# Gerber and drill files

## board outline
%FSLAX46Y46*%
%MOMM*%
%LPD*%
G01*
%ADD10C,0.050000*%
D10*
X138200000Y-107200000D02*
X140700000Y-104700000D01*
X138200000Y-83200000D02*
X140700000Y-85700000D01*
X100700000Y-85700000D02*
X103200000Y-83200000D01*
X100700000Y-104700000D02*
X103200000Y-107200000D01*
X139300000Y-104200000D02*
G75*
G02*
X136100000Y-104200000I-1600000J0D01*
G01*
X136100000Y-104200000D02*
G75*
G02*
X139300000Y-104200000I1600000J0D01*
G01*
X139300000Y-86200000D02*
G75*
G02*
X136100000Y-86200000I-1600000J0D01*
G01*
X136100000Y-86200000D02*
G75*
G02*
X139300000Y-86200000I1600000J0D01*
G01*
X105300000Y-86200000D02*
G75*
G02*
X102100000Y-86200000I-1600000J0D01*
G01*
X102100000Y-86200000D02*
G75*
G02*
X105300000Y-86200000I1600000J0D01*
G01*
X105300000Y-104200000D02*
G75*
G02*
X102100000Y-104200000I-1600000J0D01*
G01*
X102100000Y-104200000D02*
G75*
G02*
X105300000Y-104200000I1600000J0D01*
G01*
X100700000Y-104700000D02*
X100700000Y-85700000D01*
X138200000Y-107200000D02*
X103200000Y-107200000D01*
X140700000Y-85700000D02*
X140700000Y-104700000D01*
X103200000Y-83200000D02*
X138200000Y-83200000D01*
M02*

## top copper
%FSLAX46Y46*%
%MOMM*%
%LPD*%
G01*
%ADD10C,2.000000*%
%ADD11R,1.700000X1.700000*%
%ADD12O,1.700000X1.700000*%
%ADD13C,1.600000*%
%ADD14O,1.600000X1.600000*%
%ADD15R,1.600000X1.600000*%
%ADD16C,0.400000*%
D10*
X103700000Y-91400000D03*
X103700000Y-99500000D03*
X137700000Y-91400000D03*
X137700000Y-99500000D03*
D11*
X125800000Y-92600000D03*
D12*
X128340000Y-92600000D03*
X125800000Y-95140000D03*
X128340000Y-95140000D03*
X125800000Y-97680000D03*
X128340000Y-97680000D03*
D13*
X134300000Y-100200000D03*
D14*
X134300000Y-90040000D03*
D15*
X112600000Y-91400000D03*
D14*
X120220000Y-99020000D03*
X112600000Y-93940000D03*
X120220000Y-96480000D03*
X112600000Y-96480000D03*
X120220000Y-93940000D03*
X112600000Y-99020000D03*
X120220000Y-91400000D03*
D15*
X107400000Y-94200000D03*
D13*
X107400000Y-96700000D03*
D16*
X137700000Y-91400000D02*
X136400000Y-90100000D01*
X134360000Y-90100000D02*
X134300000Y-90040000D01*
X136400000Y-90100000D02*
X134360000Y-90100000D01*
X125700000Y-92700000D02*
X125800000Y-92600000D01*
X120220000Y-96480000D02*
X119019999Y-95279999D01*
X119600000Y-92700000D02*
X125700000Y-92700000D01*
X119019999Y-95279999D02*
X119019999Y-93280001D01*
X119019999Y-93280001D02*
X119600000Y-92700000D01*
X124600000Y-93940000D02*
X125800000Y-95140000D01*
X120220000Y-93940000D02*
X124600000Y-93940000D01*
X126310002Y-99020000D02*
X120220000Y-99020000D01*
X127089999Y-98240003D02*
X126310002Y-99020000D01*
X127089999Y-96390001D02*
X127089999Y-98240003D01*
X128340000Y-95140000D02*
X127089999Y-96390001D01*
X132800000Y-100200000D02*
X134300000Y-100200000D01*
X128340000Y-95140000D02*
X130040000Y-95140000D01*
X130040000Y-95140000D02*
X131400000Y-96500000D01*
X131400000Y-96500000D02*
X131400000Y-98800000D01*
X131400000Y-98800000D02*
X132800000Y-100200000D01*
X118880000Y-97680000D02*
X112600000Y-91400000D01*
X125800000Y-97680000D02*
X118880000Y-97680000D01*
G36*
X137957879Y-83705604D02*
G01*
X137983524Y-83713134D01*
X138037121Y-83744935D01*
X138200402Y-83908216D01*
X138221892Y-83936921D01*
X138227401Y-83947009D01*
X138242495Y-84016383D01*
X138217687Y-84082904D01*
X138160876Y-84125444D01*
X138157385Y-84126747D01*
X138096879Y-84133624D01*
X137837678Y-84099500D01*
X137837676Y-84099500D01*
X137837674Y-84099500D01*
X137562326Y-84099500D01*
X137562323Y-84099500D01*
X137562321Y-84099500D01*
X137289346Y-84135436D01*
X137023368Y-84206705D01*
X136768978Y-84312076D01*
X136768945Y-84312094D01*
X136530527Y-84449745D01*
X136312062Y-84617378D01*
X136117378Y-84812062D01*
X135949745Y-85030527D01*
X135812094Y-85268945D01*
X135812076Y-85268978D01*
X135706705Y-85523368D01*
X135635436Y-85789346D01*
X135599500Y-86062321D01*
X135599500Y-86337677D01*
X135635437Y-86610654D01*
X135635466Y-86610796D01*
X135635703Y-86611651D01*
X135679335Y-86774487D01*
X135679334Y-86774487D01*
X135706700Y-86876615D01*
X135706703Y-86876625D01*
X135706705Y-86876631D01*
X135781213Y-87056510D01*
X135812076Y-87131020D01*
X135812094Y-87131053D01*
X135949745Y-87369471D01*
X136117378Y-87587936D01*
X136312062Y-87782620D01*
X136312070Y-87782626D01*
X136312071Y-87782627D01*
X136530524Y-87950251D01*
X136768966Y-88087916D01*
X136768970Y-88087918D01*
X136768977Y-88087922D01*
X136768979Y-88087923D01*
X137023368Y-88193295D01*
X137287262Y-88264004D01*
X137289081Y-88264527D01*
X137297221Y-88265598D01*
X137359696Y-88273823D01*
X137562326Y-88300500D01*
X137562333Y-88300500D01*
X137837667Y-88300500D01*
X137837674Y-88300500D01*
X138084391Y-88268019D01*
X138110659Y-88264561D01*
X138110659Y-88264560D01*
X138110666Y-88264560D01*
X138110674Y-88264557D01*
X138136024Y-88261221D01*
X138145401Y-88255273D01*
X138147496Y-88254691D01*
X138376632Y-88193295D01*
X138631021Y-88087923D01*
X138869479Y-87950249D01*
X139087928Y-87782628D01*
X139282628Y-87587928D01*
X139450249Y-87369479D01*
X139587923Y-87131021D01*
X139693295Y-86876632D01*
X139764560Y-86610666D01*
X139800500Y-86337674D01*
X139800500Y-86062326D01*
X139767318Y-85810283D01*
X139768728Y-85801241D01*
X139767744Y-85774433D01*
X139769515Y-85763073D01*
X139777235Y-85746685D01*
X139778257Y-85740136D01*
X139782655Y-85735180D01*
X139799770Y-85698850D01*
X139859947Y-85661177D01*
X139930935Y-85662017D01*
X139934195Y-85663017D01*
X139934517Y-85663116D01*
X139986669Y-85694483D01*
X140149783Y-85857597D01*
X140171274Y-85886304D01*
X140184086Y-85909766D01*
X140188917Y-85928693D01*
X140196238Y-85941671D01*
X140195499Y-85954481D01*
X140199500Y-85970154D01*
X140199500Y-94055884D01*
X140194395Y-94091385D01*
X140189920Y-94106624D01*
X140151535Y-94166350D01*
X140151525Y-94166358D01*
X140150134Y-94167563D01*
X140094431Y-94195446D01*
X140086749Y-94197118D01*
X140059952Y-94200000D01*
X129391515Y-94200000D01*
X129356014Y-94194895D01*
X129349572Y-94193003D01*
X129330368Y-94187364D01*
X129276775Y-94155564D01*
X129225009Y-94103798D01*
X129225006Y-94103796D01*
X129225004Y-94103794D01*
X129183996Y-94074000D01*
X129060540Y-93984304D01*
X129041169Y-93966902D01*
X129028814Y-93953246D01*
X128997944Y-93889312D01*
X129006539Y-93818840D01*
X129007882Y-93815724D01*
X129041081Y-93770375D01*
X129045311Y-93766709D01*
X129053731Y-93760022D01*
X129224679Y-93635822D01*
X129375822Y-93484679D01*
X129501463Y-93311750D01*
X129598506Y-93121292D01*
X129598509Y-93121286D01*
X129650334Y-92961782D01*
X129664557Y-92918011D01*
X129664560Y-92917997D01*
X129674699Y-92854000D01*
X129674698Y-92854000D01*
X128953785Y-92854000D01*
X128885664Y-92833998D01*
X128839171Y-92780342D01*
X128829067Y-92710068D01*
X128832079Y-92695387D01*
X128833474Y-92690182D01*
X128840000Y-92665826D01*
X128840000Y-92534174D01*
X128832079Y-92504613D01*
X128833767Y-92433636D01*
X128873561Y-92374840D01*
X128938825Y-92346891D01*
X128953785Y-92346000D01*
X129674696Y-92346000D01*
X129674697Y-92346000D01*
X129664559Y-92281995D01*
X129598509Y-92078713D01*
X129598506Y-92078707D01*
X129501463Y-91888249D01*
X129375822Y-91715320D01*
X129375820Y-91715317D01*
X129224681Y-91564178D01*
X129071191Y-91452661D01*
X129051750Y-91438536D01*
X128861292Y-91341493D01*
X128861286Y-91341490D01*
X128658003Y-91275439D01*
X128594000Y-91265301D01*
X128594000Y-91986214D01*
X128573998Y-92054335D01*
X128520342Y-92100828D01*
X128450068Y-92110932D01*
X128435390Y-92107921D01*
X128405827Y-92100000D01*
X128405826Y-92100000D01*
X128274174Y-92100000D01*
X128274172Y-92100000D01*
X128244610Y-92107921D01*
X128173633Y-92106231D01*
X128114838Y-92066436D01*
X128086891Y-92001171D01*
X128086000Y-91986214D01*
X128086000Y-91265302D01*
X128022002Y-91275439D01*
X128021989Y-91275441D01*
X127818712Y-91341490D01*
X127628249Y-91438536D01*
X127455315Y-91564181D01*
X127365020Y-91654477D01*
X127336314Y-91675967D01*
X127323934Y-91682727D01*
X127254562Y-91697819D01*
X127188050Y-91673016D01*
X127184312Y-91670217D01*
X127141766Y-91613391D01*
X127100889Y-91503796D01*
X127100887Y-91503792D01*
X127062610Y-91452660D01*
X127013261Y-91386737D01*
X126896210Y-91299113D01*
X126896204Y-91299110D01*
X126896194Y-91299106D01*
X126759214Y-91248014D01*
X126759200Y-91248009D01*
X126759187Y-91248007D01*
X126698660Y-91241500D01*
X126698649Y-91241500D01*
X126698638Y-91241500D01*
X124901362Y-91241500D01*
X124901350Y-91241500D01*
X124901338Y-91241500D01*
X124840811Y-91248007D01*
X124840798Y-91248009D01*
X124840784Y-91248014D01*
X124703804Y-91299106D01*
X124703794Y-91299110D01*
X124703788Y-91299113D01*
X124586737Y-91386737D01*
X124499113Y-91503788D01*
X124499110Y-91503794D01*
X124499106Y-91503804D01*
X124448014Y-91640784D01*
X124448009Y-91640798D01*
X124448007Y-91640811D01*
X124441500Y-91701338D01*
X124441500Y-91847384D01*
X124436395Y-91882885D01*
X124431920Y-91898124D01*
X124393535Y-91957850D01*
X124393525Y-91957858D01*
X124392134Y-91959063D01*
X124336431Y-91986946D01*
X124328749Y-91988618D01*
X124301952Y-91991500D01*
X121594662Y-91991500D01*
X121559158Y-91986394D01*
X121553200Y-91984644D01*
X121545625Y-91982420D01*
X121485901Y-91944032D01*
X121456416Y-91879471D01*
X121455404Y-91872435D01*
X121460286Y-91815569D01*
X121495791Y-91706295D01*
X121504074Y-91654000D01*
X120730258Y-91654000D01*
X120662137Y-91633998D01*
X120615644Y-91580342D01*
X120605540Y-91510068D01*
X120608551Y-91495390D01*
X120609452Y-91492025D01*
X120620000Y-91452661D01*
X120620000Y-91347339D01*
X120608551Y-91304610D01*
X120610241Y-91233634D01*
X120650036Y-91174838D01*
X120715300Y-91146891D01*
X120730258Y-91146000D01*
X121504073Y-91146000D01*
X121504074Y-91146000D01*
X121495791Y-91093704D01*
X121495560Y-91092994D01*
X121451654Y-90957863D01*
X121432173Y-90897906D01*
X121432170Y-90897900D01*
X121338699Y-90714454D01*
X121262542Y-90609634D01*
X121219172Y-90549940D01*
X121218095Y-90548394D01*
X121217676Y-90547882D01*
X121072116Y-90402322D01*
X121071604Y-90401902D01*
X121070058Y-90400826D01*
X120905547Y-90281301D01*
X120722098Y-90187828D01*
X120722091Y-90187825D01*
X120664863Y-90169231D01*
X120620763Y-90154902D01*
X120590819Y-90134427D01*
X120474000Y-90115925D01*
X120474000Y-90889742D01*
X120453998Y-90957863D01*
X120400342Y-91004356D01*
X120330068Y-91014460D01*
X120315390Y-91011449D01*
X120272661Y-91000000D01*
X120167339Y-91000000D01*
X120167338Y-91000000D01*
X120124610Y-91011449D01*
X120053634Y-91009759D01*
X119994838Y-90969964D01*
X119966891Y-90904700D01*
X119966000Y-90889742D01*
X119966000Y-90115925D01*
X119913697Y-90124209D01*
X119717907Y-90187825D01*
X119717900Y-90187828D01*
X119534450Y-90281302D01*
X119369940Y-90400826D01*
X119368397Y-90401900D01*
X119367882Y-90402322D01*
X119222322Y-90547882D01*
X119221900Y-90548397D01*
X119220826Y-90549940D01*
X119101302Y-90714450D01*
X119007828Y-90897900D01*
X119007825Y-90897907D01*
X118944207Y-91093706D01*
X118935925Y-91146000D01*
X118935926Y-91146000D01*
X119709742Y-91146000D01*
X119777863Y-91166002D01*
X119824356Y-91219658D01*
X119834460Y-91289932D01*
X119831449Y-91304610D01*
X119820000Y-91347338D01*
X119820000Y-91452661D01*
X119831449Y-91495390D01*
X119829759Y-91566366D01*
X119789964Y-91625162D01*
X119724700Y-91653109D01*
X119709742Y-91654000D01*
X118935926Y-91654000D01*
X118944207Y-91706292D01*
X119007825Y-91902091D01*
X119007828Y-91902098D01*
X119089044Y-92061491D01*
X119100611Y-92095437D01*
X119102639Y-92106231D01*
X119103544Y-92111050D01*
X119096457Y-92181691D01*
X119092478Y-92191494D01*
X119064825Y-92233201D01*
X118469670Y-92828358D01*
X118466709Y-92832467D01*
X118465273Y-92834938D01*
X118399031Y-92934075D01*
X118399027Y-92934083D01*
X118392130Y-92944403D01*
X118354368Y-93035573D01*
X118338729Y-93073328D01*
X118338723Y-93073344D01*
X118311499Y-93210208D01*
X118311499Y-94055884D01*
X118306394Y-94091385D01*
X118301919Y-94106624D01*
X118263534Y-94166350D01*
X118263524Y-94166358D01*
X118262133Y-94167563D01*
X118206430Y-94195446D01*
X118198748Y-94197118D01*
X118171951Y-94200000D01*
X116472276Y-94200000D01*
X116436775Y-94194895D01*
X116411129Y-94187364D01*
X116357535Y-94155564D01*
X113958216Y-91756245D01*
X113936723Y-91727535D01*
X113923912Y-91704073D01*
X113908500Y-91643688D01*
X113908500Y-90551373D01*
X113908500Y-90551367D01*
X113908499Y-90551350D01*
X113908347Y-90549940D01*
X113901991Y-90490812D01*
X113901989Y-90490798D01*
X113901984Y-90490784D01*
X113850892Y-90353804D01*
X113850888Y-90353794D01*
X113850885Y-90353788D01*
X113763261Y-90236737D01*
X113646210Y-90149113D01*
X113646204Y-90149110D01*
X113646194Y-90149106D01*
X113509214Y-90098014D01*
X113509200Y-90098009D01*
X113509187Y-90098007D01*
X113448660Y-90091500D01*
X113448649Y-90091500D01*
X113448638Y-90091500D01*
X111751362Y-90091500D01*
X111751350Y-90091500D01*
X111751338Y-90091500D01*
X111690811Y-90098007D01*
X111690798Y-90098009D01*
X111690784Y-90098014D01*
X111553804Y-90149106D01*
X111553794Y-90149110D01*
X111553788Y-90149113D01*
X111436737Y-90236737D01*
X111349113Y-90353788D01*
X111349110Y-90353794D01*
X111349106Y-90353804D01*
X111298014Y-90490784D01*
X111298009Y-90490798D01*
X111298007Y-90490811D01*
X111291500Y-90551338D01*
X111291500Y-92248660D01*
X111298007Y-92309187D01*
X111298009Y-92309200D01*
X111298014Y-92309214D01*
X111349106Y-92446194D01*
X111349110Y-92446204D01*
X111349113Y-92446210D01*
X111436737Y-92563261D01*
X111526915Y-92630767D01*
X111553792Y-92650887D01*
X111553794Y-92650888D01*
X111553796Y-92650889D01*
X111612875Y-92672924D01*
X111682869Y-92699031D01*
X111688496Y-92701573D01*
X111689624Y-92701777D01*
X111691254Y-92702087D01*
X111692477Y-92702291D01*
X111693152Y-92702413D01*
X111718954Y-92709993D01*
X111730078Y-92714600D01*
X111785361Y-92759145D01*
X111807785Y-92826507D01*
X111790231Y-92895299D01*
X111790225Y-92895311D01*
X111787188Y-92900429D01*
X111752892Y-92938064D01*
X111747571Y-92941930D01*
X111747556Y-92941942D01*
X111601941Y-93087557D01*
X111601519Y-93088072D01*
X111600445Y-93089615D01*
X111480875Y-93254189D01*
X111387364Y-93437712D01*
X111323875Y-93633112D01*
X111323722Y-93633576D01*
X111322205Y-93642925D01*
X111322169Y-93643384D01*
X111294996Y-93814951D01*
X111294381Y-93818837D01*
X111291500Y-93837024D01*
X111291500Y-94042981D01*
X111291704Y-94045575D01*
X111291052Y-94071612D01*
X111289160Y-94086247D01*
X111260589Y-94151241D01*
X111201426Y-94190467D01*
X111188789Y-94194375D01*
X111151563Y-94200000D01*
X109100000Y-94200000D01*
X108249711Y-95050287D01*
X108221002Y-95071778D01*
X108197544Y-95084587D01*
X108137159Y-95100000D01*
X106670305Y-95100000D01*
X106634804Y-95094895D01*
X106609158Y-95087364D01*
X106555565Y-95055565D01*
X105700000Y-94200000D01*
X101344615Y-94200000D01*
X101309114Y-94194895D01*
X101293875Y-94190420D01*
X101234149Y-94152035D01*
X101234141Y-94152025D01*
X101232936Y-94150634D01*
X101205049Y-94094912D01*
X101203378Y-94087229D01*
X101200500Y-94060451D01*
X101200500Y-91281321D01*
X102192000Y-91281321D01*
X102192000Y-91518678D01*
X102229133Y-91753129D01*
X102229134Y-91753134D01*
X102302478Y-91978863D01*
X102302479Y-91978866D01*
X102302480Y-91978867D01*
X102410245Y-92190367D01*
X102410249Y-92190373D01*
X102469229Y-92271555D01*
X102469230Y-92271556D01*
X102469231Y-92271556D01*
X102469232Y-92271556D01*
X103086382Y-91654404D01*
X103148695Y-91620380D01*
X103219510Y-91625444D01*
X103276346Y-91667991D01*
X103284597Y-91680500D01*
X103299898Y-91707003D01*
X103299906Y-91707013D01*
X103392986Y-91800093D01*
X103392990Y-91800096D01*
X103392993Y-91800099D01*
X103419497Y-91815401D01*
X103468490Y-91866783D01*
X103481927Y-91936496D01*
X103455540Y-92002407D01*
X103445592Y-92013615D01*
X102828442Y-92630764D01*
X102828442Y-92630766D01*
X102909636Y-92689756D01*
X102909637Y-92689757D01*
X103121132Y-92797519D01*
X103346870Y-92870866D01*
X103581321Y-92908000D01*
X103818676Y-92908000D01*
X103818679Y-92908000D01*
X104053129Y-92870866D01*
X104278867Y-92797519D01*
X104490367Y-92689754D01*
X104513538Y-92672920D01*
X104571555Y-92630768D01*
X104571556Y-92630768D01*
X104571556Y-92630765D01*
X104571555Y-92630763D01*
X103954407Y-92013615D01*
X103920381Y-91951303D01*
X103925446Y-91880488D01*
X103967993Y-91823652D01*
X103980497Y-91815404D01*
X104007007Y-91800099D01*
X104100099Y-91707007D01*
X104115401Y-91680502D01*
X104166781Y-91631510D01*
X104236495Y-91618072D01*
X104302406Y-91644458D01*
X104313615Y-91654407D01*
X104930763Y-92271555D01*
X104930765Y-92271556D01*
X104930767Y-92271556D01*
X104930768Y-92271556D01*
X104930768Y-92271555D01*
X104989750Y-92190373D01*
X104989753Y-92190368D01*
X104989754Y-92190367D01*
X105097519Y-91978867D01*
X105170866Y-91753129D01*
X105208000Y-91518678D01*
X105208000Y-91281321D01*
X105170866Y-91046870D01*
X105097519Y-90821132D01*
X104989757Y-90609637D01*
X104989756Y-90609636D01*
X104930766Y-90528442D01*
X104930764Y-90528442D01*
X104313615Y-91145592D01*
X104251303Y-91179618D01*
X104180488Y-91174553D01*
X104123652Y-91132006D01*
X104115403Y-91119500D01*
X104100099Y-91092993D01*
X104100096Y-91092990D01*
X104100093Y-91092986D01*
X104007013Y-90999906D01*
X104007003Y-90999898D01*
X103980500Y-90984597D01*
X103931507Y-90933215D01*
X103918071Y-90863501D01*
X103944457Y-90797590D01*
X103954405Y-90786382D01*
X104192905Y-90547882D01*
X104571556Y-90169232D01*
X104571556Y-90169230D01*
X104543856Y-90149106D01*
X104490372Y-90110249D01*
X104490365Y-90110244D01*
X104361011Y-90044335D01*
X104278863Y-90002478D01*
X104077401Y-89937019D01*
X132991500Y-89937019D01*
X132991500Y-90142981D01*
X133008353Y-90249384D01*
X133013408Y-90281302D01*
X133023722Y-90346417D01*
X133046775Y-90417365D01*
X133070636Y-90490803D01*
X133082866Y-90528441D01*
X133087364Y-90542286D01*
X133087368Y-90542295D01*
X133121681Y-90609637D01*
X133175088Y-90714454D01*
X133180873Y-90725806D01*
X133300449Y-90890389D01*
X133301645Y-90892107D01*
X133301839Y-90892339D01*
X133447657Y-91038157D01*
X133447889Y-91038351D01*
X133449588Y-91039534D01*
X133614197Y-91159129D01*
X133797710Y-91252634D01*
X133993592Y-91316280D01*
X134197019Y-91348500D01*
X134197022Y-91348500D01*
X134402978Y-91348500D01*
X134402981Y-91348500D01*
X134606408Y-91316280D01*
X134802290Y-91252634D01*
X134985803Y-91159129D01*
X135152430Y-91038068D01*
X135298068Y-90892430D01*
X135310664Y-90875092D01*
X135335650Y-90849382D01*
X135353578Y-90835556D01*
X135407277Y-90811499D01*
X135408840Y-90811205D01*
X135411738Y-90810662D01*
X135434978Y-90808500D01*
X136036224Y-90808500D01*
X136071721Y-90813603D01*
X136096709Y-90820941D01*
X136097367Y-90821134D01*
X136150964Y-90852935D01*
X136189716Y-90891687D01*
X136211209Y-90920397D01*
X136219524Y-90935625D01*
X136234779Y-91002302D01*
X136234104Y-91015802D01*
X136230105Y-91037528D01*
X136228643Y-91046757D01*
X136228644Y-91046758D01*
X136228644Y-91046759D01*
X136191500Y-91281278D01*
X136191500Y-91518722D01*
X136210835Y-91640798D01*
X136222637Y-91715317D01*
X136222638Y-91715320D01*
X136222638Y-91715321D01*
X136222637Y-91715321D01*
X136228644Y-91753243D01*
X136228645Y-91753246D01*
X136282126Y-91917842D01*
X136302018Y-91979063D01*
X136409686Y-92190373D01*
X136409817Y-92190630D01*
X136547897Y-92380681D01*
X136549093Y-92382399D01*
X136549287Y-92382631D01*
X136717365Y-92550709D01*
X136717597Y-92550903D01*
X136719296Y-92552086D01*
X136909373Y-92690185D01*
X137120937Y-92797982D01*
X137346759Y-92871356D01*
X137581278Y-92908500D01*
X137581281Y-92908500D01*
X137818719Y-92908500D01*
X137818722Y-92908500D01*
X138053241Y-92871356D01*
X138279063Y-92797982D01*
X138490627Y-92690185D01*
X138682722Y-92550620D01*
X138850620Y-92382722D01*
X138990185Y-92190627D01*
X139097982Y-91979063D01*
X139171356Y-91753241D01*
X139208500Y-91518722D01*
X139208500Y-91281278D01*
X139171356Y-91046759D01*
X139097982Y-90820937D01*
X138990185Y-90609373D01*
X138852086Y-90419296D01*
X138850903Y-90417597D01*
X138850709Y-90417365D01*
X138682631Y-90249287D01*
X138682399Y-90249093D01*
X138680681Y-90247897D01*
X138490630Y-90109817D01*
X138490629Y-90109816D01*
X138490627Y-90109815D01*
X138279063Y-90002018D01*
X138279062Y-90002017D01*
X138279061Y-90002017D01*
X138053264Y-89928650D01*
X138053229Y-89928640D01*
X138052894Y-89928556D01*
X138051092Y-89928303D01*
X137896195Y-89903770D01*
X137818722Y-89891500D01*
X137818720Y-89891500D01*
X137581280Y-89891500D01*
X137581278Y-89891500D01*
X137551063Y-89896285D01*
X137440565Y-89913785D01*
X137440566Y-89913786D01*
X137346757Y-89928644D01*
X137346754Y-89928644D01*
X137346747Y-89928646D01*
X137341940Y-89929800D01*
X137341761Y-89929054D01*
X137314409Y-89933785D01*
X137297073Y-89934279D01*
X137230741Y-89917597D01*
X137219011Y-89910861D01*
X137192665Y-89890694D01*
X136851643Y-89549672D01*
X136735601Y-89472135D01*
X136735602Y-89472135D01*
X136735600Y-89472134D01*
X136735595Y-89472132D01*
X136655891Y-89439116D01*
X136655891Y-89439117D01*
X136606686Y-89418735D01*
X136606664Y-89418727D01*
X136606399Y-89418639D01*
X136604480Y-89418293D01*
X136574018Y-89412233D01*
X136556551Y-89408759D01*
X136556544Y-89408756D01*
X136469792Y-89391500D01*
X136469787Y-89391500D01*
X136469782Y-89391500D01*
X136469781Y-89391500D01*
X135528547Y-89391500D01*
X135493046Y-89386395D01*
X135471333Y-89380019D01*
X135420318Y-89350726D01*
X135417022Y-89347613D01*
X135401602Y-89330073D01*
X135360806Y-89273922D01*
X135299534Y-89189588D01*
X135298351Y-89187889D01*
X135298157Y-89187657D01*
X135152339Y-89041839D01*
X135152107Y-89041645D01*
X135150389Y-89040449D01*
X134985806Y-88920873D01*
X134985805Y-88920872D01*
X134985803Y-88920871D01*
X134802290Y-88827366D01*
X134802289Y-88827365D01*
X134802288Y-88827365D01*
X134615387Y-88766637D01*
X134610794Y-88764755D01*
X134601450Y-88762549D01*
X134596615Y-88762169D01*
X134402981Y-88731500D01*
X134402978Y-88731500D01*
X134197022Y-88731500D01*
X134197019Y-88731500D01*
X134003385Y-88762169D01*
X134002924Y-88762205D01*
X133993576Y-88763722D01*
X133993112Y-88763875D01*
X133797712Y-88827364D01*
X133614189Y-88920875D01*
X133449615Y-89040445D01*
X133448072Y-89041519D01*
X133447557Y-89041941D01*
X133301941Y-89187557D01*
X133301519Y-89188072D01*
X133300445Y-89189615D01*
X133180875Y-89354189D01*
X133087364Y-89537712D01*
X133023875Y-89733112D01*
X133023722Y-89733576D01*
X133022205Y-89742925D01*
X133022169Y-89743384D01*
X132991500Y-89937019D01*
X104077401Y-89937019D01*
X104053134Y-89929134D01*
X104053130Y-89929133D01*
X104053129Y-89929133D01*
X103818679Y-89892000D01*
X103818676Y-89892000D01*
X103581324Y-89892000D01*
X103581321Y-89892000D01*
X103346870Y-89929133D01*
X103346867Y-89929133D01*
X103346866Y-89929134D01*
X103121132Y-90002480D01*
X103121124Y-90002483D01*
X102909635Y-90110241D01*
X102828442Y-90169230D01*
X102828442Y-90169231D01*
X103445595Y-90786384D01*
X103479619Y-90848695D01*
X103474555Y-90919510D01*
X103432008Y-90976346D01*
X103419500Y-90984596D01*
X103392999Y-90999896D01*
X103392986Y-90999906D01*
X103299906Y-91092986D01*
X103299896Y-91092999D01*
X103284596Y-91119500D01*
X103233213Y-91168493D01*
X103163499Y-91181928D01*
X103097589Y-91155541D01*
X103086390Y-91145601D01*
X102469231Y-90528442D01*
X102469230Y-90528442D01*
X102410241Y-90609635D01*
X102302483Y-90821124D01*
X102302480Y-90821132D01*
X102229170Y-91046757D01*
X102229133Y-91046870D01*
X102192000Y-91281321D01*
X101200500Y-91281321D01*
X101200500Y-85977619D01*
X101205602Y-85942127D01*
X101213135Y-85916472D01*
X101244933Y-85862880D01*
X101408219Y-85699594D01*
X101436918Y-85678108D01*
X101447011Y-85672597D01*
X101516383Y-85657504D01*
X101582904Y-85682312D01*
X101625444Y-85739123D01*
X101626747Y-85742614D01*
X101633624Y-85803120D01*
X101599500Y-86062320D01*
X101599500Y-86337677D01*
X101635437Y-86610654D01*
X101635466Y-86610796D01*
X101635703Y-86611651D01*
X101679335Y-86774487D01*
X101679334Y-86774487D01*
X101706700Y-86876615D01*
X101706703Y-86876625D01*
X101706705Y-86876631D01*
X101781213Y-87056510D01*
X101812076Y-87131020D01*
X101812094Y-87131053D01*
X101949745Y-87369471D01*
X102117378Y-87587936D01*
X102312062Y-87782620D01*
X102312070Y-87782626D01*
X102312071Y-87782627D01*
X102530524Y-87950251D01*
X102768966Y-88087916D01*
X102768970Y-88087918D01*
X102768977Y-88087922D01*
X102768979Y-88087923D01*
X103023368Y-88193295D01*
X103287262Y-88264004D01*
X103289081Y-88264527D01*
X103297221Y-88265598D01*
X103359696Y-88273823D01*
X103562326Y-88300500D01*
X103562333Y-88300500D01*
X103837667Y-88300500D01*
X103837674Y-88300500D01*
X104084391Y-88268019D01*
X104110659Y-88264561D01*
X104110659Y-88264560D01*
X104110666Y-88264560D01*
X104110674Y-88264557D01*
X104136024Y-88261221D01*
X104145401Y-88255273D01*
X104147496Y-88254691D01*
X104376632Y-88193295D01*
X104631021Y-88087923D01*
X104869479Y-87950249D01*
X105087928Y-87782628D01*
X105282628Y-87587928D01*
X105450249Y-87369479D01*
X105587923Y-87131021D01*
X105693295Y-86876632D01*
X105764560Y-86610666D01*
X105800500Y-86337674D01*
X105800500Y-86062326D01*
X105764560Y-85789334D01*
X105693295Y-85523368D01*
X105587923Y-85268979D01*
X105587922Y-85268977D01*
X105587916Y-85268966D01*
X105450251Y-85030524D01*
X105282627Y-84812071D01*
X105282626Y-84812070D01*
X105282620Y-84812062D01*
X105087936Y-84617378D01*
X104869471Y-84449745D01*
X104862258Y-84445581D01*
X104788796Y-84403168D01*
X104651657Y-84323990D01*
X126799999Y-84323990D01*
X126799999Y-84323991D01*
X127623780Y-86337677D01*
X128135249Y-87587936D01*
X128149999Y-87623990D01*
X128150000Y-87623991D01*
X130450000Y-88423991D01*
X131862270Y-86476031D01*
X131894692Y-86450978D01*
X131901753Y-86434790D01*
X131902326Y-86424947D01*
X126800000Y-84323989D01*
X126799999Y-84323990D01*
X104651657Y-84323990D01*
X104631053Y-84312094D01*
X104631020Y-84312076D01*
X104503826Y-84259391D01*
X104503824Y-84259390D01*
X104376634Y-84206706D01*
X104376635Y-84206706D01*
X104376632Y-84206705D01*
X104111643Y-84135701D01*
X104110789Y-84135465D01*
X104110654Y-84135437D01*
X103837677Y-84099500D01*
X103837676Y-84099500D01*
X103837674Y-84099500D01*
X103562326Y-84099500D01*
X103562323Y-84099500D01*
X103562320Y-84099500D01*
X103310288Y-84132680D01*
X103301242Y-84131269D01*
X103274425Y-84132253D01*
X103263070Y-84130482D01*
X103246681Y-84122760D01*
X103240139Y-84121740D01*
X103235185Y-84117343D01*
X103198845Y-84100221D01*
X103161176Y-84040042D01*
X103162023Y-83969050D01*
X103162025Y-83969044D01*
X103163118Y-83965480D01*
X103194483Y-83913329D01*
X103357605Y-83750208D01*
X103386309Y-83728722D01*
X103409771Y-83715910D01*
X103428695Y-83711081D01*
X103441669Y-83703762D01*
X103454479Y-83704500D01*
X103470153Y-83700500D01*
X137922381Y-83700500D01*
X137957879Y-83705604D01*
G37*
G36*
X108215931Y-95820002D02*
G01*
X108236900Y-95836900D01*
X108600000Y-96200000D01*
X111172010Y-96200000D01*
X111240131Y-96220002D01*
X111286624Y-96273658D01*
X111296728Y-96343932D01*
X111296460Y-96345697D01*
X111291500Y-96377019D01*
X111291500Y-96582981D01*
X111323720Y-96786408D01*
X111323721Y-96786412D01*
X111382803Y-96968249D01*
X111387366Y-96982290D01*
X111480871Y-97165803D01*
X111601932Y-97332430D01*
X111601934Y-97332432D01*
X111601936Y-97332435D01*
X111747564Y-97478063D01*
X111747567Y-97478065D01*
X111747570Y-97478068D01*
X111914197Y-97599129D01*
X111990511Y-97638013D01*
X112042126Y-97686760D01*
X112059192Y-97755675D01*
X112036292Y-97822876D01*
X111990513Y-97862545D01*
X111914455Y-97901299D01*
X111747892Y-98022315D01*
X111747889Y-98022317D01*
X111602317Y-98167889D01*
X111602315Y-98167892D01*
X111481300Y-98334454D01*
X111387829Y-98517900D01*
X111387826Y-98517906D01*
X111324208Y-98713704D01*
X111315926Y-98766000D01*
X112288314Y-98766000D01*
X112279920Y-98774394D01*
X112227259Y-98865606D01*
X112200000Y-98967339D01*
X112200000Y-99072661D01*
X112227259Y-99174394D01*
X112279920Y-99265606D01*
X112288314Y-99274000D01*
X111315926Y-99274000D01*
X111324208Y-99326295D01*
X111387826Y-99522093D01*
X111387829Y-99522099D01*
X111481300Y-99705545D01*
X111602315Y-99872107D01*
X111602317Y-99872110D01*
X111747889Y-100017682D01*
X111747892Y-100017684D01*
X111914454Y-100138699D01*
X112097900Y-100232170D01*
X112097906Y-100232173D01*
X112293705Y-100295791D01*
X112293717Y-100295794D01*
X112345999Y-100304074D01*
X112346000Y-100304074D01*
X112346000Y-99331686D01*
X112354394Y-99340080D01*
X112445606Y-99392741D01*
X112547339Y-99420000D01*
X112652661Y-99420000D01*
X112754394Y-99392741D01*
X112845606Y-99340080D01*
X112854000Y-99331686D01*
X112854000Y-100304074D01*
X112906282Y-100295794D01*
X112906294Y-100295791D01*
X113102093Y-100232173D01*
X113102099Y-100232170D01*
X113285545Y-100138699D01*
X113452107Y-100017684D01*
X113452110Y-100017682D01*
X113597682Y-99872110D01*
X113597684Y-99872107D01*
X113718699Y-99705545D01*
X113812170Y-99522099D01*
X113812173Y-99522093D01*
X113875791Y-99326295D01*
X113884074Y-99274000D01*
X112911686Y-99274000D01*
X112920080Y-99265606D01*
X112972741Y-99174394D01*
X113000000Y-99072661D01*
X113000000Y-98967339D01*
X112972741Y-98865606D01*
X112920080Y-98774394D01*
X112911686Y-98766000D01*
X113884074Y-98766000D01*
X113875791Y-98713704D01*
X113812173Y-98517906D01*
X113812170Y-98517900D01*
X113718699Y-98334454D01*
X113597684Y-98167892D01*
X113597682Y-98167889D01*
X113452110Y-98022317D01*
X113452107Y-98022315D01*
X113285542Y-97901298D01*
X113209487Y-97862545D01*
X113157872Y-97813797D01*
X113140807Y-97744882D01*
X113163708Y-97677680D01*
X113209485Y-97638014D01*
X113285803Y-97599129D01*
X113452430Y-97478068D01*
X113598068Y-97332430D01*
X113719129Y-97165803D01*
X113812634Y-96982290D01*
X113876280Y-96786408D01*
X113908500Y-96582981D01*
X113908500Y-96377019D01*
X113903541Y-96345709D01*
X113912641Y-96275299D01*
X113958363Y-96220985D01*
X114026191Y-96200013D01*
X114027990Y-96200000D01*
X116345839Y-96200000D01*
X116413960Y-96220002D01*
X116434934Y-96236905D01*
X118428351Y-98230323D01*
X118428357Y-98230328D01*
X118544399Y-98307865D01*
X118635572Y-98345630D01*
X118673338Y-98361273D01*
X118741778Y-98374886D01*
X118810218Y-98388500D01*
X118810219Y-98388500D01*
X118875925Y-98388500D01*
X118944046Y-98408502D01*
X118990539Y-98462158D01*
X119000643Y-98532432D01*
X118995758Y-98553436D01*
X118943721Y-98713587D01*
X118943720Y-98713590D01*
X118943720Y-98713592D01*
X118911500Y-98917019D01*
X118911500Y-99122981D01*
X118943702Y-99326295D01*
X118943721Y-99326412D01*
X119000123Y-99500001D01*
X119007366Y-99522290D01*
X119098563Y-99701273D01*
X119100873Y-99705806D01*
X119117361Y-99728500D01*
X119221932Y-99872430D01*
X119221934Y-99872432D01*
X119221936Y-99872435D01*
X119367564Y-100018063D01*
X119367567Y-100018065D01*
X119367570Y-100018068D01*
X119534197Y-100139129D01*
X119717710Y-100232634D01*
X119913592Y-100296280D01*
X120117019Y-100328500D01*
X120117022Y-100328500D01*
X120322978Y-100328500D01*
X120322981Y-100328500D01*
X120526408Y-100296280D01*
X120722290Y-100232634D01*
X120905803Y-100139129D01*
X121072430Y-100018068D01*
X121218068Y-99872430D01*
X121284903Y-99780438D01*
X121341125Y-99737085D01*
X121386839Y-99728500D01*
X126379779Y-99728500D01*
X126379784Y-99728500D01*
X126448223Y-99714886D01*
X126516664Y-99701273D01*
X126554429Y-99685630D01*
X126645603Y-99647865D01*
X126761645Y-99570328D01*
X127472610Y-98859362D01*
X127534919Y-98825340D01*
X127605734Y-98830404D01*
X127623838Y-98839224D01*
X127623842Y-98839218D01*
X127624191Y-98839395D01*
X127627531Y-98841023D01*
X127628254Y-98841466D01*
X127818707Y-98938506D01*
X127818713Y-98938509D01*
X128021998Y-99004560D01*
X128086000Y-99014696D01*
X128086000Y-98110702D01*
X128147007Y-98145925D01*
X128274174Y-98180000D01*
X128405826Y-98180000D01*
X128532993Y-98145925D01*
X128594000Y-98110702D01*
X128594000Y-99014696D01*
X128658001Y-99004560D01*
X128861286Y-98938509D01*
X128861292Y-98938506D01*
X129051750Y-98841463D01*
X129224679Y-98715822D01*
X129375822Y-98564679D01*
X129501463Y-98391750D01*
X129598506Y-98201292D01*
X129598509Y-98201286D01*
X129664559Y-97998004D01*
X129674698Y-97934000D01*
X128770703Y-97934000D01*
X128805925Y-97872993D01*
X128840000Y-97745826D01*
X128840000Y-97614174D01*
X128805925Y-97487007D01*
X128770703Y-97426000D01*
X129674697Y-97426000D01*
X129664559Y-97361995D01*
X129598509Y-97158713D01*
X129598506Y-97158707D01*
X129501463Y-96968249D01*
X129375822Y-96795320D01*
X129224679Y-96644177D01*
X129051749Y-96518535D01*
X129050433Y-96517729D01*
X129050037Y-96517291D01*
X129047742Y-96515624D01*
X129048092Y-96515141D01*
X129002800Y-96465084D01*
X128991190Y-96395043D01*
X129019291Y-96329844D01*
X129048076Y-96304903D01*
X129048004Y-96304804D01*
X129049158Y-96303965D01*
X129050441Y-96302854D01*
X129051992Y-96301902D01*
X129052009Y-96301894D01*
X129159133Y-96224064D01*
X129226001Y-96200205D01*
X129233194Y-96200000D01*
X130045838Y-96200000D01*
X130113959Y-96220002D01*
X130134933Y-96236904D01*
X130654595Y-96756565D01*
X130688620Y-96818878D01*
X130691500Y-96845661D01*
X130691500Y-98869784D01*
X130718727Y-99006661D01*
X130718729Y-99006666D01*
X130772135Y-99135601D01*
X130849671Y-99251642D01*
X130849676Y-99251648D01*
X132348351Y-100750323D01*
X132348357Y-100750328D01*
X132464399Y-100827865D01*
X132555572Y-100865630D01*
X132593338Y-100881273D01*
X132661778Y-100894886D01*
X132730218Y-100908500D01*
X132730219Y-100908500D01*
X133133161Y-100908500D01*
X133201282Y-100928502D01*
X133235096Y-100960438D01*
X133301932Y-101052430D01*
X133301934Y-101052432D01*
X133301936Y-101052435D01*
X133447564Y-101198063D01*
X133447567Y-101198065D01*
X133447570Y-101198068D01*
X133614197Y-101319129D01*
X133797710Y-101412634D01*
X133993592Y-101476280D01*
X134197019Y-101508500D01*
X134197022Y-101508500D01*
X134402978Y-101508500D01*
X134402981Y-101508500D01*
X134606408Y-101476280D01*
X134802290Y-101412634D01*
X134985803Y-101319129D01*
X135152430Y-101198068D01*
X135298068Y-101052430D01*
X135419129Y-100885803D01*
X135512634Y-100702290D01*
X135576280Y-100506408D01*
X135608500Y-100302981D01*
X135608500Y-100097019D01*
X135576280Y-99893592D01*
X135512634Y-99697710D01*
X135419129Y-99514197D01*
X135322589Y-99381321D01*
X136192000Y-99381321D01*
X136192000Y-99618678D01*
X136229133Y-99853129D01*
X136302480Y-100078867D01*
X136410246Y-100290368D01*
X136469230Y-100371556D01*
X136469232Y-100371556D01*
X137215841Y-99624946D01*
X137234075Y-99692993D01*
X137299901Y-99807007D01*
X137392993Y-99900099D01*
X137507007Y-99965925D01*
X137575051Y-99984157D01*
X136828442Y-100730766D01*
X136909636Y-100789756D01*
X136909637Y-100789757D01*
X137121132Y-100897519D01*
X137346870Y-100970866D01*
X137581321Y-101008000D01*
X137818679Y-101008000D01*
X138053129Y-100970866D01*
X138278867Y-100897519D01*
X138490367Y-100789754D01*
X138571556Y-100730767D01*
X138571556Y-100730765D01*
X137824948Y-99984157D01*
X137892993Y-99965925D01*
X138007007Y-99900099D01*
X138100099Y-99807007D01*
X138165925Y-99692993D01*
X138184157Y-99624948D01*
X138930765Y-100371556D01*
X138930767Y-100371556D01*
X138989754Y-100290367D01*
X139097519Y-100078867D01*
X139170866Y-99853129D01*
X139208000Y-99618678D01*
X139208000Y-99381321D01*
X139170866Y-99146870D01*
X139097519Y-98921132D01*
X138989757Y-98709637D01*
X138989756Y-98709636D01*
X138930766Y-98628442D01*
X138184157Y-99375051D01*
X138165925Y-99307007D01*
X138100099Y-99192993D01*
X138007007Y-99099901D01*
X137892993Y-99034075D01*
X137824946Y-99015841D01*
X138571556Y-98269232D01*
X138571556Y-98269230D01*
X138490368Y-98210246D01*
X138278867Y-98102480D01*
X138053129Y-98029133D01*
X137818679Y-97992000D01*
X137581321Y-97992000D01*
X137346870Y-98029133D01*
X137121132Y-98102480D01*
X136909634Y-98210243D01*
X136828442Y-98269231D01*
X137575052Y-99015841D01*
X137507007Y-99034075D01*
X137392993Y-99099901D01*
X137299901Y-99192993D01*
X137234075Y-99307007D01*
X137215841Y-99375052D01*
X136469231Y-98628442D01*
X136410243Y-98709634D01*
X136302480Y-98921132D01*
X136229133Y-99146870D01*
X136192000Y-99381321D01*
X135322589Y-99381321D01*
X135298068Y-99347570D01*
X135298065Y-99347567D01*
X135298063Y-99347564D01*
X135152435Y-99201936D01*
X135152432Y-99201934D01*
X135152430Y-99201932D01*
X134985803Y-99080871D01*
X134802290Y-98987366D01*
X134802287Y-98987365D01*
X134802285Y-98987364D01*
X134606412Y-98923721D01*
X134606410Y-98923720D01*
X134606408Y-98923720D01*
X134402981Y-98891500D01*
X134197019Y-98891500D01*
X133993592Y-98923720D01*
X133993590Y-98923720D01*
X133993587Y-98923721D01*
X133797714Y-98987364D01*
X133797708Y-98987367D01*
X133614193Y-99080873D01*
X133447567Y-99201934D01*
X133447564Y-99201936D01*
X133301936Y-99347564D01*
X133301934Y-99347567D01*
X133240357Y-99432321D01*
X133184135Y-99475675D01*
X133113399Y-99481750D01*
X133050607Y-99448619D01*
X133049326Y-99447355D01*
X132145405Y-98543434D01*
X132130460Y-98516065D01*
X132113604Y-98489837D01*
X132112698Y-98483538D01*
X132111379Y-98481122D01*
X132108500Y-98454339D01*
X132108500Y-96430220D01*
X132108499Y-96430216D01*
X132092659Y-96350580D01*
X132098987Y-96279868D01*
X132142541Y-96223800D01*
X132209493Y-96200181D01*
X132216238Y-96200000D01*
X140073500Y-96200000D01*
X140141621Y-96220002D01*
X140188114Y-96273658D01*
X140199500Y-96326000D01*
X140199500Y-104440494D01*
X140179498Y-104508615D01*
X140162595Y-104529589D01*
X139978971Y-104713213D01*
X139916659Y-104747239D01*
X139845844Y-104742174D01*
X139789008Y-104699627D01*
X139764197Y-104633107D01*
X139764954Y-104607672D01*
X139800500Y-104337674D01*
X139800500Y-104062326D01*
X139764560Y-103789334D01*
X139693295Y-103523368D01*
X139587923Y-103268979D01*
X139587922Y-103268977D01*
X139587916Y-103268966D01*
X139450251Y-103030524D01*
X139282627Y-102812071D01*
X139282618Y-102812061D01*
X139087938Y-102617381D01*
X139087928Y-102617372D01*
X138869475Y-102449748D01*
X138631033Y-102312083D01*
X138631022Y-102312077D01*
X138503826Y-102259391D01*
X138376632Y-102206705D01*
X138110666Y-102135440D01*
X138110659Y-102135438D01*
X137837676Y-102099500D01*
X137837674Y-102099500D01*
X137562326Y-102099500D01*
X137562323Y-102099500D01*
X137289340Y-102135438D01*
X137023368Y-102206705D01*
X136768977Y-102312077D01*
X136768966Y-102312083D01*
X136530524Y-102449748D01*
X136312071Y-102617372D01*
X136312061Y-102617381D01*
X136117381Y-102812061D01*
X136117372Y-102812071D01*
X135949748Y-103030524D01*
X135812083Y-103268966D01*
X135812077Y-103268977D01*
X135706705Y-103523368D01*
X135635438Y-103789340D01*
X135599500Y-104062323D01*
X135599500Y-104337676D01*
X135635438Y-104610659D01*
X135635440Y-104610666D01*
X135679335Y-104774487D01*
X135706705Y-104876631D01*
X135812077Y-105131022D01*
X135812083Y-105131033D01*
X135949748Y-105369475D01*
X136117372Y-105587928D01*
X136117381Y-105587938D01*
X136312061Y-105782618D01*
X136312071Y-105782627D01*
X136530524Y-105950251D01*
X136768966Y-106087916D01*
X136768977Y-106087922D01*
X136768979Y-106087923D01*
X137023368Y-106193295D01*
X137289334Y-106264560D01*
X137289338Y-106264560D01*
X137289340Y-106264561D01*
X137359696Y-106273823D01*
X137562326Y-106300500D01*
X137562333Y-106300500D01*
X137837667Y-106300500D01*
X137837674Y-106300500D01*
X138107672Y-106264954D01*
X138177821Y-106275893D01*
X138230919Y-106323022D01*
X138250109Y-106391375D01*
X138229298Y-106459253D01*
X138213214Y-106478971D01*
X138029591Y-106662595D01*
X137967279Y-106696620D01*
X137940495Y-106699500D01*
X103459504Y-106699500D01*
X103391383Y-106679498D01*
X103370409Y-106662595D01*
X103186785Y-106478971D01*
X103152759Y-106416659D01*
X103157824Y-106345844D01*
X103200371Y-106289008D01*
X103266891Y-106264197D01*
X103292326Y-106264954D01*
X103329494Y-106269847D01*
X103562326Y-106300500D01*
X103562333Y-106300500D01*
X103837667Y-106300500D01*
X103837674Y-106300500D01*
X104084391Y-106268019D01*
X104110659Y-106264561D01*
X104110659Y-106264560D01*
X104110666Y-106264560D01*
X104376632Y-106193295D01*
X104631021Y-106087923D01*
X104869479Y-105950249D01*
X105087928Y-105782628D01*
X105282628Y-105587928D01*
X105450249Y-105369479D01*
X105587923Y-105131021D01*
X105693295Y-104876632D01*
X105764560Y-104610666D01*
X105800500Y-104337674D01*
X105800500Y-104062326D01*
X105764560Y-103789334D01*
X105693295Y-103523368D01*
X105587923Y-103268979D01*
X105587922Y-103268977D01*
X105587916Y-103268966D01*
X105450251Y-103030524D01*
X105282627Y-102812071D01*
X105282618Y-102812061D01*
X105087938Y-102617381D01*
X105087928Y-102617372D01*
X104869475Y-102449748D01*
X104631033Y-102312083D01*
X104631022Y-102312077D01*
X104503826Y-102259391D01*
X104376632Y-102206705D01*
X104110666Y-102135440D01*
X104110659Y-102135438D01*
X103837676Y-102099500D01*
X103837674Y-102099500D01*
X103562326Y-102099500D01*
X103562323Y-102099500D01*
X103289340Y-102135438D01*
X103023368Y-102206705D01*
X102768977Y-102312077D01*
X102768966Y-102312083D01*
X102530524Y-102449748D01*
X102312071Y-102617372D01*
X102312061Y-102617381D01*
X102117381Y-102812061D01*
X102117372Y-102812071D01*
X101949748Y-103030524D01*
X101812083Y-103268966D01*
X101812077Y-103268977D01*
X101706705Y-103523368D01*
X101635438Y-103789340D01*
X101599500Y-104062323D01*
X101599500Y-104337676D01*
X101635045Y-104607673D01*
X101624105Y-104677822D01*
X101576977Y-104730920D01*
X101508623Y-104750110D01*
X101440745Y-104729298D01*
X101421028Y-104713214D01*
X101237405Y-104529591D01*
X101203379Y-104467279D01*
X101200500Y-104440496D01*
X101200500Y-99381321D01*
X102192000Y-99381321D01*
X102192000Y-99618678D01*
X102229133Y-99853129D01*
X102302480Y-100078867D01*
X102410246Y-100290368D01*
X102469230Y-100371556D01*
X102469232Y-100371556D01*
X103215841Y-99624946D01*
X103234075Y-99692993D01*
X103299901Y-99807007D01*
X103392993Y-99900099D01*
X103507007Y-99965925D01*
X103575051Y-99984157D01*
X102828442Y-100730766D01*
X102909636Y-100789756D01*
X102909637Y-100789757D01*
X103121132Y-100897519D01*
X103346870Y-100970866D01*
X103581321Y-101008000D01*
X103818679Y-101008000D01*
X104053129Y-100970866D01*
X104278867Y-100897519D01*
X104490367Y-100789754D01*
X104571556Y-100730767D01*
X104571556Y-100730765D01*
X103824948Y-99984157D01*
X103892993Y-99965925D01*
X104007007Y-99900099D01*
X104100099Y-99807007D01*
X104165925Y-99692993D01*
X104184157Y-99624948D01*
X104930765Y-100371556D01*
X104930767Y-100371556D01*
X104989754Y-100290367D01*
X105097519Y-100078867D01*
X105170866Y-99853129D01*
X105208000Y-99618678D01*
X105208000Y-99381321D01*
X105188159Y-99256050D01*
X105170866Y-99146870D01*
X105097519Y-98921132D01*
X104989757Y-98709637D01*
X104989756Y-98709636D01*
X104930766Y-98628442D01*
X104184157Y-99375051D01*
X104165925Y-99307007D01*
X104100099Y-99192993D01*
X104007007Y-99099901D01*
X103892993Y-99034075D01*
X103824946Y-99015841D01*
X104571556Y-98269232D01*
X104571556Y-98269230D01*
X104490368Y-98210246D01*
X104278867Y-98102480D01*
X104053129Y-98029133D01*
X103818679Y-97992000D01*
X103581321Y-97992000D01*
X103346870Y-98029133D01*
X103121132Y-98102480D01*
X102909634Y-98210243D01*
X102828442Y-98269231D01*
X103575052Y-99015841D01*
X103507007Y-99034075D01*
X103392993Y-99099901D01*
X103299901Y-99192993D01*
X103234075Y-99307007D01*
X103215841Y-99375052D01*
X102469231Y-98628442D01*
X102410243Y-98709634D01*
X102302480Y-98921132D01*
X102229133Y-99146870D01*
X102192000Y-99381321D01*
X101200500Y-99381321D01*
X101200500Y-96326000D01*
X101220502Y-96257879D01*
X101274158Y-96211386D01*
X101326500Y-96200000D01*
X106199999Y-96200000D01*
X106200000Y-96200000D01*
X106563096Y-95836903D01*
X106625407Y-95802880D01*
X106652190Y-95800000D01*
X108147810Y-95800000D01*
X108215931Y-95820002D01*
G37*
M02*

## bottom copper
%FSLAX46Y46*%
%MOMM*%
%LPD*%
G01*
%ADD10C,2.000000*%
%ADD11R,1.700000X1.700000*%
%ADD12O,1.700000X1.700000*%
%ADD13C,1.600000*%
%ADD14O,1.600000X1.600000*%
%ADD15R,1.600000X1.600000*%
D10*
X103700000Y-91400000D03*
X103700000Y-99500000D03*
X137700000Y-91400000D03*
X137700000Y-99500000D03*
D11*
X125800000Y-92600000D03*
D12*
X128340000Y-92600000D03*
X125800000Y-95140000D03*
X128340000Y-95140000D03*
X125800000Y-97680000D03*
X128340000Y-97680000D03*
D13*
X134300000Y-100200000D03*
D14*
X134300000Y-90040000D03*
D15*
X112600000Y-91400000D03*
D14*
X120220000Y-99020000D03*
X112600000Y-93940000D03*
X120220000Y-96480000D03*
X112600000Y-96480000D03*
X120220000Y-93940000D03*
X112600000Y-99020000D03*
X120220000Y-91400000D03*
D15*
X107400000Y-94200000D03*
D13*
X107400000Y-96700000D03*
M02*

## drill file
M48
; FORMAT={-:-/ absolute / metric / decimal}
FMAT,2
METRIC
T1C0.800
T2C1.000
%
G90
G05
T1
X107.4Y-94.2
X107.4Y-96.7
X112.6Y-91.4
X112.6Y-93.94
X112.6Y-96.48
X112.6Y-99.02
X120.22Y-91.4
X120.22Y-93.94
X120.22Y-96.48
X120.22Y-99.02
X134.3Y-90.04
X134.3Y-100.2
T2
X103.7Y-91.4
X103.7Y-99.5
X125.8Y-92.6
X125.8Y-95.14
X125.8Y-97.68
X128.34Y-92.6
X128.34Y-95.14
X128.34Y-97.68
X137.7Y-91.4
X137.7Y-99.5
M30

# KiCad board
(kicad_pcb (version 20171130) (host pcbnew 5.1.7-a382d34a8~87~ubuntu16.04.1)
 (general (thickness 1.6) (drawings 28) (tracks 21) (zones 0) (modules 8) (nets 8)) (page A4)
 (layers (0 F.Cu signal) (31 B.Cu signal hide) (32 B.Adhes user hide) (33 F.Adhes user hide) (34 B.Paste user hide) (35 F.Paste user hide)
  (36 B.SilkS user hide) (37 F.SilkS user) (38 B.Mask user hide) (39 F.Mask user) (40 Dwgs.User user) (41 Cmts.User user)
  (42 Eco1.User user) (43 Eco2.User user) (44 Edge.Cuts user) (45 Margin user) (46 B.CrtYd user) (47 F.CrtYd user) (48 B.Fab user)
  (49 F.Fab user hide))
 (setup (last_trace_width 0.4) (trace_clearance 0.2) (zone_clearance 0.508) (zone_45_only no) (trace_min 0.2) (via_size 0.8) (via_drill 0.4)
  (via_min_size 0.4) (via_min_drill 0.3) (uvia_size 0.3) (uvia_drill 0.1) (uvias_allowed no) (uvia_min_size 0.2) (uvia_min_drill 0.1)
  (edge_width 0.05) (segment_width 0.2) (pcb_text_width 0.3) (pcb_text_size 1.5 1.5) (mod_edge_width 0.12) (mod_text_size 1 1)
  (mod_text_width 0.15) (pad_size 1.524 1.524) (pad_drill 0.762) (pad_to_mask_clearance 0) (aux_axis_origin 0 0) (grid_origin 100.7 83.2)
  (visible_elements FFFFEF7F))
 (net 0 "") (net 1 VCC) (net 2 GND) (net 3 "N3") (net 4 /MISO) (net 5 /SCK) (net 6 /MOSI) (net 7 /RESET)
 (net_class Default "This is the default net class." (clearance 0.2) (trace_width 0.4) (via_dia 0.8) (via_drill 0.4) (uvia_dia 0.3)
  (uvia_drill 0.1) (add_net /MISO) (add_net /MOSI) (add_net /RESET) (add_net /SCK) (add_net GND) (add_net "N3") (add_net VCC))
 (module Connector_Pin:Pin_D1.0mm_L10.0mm (layer F.Cu) (at 103.7 91.4)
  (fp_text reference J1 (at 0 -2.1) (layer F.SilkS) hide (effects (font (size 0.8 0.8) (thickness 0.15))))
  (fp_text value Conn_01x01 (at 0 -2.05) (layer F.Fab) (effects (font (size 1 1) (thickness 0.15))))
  (pad 1 thru_hole circle (at 0 0) (size 2 2) (drill 1) (layers *.Cu *.Mask) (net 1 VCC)))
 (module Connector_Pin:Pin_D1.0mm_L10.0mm (layer F.Cu) (at 103.7 99.5)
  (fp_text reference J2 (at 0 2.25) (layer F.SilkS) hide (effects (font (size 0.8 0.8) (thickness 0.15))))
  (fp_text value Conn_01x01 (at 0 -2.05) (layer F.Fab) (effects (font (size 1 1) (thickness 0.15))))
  (pad 1 thru_hole circle (at 0 0) (size 2 2) (drill 1) (layers *.Cu *.Mask) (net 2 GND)))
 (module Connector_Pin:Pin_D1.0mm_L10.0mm (layer F.Cu) (at 137.7 91.4)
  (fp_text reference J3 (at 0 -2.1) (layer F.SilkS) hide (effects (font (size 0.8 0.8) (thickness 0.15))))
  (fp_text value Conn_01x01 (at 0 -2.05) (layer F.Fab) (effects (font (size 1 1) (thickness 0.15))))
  (pad 1 thru_hole circle (at 0 0) (size 2 2) (drill 1) (layers *.Cu *.Mask) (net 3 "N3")))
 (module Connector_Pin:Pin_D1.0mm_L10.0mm (layer F.Cu) (at 137.7 99.5)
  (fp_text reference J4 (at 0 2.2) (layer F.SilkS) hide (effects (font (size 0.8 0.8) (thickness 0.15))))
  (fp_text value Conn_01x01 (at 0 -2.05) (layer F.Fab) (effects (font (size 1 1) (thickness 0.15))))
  (pad 1 thru_hole circle (at 0 0) (size 2 2) (drill 1) (layers *.Cu *.Mask) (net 2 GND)))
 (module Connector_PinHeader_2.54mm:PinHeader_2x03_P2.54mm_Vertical (layer F.Cu) (at 125.8 92.6)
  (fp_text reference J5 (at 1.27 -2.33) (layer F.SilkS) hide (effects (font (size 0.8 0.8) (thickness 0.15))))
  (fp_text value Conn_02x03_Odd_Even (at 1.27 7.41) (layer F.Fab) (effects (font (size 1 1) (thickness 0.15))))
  (pad 1 thru_hole rect (at 0 0) (size 1.7 1.7) (drill 1) (layers *.Cu *.Mask) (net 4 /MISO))
  (pad 2 thru_hole oval (at 2.54 0) (size 1.7 1.7) (drill 1) (layers *.Cu *.Mask) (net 1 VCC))
  (pad 3 thru_hole oval (at 0 2.54) (size 1.7 1.7) (drill 1) (layers *.Cu *.Mask) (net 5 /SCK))
  (pad 4 thru_hole oval (at 2.54 2.54) (size 1.7 1.7) (drill 1) (layers *.Cu *.Mask) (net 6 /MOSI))
  (pad 5 thru_hole oval (at 0 5.08) (size 1.7 1.7) (drill 1) (layers *.Cu *.Mask) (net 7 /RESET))
  (pad 6 thru_hole oval (at 2.54 5.08) (size 1.7 1.7) (drill 1) (layers *.Cu *.Mask) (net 2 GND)))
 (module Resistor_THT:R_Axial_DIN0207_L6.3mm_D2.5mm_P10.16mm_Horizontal (layer F.Cu) (at 134.3 100.2 90)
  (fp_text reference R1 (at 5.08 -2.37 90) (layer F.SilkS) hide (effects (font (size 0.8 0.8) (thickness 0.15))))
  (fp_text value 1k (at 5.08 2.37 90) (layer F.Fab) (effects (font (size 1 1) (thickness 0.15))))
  (pad 1 thru_hole circle (at 0 0 90) (size 1.6 1.6) (drill 0.8) (layers *.Cu *.Mask) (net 6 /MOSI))
  (pad 2 thru_hole oval (at 10.16 0 90) (size 1.6 1.6) (drill 0.8) (layers *.Cu *.Mask) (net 3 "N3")))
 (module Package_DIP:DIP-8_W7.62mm (layer F.Cu) (at 112.6 91.4)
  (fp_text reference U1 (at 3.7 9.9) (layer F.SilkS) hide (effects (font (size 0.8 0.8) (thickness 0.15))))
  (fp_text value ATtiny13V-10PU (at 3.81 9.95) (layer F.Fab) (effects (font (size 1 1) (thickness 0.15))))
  (pad 1 thru_hole rect (at 0 0) (size 1.6 1.6) (drill 0.8) (layers *.Cu *.Mask) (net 7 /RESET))
  (pad 5 thru_hole oval (at 7.62 7.62) (size 1.6 1.6) (drill 0.8) (layers *.Cu *.Mask) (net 6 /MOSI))
  (pad 2 thru_hole oval (at 0 2.54) (size 1.6 1.6) (drill 0.8) (layers *.Cu *.Mask))
  (pad 6 thru_hole oval (at 7.62 5.08) (size 1.6 1.6) (drill 0.8) (layers *.Cu *.Mask) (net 4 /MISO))
  (pad 3 thru_hole oval (at 0 5.08) (size 1.6 1.6) (drill 0.8) (layers *.Cu *.Mask))
  (pad 7 thru_hole oval (at 7.62 2.54) (size 1.6 1.6) (drill 0.8) (layers *.Cu *.Mask) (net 5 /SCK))
  (pad 4 thru_hole oval (at 0 7.62) (size 1.6 1.6) (drill 0.8) (layers *.Cu *.Mask) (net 2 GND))
  (pad 8 thru_hole oval (at 7.62 0) (size 1.6 1.6) (drill 0.8) (layers *.Cu *.Mask) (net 1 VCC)))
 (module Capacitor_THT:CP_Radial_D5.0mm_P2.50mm (layer F.Cu) (at 107.4 94.2 270) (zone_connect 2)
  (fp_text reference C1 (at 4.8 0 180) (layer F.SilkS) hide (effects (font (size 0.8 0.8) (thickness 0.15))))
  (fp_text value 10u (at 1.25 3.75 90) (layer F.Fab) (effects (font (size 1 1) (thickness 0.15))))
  (pad 1 thru_hole rect (at 0 0 270) (size 1.6 1.6) (drill 0.8) (layers *.Cu *.Mask) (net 1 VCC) (zone_connect 2))
  (pad 2 thru_hole circle (at 2.5 0 270) (size 1.6 1.6) (drill 0.8) (layers *.Cu *.Mask) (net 2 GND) (zone_connect 2)))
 (gr_line (start 138.2 107.2) (end 140.7 104.7) (layer Edge.Cuts) (width 0.05))
 (gr_line (start 138.2 83.2) (end 140.7 85.7) (layer Edge.Cuts) (width 0.05))
 (gr_line (start 100.7 85.7) (end 103.2 83.2) (layer Edge.Cuts) (width 0.05))
 (gr_line (start 100.7 104.7) (end 103.2 107.2) (layer Edge.Cuts) (width 0.05))
 (gr_circle (center 137.7 104.2) (end 139.3 104.2) (layer Edge.Cuts) (width 0.05))
 (gr_circle (center 137.7 86.2) (end 139.3 86.2) (layer Edge.Cuts) (width 0.05))
 (gr_circle (center 103.7 86.2) (end 105.3 86.2) (layer Edge.Cuts) (width 0.05))
 (gr_circle (center 103.7 104.2) (end 105.3 104.2) (layer Edge.Cuts) (width 0.05))
 (gr_line (start 100.7 104.7) (end 100.7 85.7) (layer Edge.Cuts) (width 0.05))
 (gr_line (start 138.2 107.2) (end 103.2 107.2) (layer Edge.Cuts) (width 0.05))
 (gr_line (start 140.7 85.7) (end 140.7 104.7) (layer Edge.Cuts) (width 0.05))
 (gr_line (start 103.2 83.2) (end 138.2 83.2) (layer Edge.Cuts) (width 0.05))
 (segment (start 137.7 91.4) (end 136.4 90.1) (width 0.4) (layer F.Cu) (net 3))
 (segment (start 134.36 90.1) (end 134.3 90.04) (width 0.4) (layer F.Cu) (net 3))
 (segment (start 136.4 90.1) (end 134.36 90.1) (width 0.4) (layer F.Cu) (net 3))
 (segment (start 125.7 92.7) (end 125.8 92.6) (width 0.4) (layer F.Cu) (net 4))
 (segment (start 120.22 96.48) (end 119.019999 95.279999) (width 0.4) (layer F.Cu) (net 4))
 (segment (start 119.6 92.7) (end 125.7 92.7) (width 0.4) (layer F.Cu) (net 4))
 (segment (start 119.019999 95.279999) (end 119.019999 93.280001) (width 0.4) (layer F.Cu) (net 4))
 (segment (start 119.019999 93.280001) (end 119.6 92.7) (width 0.4) (layer F.Cu) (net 4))
 (segment (start 124.6 93.94) (end 125.8 95.14) (width 0.4) (layer F.Cu) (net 5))
 (segment (start 120.22 93.94) (end 124.6 93.94) (width 0.4) (layer F.Cu) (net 5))
 (segment (start 126.310002 99.02) (end 120.22 99.02) (width 0.4) (layer F.Cu) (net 6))
 (segment (start 127.089999 98.240003) (end 126.310002 99.02) (width 0.4) (layer F.Cu) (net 6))
 (segment (start 127.089999 96.390001) (end 127.089999 98.240003) (width 0.4) (layer F.Cu) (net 6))
 (segment (start 128.34 95.14) (end 127.089999 96.390001) (width 0.4) (layer F.Cu) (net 6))
 (segment (start 132.8 100.2) (end 134.3 100.2) (width 0.4) (layer F.Cu) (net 6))
 (segment (start 128.34 95.14) (end 130.04 95.14) (width 0.4) (layer F.Cu) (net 6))
 (segment (start 130.04 95.14) (end 131.4 96.5) (width 0.4) (layer F.Cu) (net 6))
 (segment (start 131.4 96.5) (end 131.4 98.8) (width 0.4) (layer F.Cu) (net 6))
 (segment (start 131.4 98.8) (end 132.8 100.2) (width 0.4) (layer F.Cu) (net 6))
 (segment (start 118.88 97.68) (end 112.6 91.4) (width 0.4) (layer F.Cu) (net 7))
 (segment (start 125.8 97.68) (end 118.88 97.68) (width 0.4) (layer F.Cu) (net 7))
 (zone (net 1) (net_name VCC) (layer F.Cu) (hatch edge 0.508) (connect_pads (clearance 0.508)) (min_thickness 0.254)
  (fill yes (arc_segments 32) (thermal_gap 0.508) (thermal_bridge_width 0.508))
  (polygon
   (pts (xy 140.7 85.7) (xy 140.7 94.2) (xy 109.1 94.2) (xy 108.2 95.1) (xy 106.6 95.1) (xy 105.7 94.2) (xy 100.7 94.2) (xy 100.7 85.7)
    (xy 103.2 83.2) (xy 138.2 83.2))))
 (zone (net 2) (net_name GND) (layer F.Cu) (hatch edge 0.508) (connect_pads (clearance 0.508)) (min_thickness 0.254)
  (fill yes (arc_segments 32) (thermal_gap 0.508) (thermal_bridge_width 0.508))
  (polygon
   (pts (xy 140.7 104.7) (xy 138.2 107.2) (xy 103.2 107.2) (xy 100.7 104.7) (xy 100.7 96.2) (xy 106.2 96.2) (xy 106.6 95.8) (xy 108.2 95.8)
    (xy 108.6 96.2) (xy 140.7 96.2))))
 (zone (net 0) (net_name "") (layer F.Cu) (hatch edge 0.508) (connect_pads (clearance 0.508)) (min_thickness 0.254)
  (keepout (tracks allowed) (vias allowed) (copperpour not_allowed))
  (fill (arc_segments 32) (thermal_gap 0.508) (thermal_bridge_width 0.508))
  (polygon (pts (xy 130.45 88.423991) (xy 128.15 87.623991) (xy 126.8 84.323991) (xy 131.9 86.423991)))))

